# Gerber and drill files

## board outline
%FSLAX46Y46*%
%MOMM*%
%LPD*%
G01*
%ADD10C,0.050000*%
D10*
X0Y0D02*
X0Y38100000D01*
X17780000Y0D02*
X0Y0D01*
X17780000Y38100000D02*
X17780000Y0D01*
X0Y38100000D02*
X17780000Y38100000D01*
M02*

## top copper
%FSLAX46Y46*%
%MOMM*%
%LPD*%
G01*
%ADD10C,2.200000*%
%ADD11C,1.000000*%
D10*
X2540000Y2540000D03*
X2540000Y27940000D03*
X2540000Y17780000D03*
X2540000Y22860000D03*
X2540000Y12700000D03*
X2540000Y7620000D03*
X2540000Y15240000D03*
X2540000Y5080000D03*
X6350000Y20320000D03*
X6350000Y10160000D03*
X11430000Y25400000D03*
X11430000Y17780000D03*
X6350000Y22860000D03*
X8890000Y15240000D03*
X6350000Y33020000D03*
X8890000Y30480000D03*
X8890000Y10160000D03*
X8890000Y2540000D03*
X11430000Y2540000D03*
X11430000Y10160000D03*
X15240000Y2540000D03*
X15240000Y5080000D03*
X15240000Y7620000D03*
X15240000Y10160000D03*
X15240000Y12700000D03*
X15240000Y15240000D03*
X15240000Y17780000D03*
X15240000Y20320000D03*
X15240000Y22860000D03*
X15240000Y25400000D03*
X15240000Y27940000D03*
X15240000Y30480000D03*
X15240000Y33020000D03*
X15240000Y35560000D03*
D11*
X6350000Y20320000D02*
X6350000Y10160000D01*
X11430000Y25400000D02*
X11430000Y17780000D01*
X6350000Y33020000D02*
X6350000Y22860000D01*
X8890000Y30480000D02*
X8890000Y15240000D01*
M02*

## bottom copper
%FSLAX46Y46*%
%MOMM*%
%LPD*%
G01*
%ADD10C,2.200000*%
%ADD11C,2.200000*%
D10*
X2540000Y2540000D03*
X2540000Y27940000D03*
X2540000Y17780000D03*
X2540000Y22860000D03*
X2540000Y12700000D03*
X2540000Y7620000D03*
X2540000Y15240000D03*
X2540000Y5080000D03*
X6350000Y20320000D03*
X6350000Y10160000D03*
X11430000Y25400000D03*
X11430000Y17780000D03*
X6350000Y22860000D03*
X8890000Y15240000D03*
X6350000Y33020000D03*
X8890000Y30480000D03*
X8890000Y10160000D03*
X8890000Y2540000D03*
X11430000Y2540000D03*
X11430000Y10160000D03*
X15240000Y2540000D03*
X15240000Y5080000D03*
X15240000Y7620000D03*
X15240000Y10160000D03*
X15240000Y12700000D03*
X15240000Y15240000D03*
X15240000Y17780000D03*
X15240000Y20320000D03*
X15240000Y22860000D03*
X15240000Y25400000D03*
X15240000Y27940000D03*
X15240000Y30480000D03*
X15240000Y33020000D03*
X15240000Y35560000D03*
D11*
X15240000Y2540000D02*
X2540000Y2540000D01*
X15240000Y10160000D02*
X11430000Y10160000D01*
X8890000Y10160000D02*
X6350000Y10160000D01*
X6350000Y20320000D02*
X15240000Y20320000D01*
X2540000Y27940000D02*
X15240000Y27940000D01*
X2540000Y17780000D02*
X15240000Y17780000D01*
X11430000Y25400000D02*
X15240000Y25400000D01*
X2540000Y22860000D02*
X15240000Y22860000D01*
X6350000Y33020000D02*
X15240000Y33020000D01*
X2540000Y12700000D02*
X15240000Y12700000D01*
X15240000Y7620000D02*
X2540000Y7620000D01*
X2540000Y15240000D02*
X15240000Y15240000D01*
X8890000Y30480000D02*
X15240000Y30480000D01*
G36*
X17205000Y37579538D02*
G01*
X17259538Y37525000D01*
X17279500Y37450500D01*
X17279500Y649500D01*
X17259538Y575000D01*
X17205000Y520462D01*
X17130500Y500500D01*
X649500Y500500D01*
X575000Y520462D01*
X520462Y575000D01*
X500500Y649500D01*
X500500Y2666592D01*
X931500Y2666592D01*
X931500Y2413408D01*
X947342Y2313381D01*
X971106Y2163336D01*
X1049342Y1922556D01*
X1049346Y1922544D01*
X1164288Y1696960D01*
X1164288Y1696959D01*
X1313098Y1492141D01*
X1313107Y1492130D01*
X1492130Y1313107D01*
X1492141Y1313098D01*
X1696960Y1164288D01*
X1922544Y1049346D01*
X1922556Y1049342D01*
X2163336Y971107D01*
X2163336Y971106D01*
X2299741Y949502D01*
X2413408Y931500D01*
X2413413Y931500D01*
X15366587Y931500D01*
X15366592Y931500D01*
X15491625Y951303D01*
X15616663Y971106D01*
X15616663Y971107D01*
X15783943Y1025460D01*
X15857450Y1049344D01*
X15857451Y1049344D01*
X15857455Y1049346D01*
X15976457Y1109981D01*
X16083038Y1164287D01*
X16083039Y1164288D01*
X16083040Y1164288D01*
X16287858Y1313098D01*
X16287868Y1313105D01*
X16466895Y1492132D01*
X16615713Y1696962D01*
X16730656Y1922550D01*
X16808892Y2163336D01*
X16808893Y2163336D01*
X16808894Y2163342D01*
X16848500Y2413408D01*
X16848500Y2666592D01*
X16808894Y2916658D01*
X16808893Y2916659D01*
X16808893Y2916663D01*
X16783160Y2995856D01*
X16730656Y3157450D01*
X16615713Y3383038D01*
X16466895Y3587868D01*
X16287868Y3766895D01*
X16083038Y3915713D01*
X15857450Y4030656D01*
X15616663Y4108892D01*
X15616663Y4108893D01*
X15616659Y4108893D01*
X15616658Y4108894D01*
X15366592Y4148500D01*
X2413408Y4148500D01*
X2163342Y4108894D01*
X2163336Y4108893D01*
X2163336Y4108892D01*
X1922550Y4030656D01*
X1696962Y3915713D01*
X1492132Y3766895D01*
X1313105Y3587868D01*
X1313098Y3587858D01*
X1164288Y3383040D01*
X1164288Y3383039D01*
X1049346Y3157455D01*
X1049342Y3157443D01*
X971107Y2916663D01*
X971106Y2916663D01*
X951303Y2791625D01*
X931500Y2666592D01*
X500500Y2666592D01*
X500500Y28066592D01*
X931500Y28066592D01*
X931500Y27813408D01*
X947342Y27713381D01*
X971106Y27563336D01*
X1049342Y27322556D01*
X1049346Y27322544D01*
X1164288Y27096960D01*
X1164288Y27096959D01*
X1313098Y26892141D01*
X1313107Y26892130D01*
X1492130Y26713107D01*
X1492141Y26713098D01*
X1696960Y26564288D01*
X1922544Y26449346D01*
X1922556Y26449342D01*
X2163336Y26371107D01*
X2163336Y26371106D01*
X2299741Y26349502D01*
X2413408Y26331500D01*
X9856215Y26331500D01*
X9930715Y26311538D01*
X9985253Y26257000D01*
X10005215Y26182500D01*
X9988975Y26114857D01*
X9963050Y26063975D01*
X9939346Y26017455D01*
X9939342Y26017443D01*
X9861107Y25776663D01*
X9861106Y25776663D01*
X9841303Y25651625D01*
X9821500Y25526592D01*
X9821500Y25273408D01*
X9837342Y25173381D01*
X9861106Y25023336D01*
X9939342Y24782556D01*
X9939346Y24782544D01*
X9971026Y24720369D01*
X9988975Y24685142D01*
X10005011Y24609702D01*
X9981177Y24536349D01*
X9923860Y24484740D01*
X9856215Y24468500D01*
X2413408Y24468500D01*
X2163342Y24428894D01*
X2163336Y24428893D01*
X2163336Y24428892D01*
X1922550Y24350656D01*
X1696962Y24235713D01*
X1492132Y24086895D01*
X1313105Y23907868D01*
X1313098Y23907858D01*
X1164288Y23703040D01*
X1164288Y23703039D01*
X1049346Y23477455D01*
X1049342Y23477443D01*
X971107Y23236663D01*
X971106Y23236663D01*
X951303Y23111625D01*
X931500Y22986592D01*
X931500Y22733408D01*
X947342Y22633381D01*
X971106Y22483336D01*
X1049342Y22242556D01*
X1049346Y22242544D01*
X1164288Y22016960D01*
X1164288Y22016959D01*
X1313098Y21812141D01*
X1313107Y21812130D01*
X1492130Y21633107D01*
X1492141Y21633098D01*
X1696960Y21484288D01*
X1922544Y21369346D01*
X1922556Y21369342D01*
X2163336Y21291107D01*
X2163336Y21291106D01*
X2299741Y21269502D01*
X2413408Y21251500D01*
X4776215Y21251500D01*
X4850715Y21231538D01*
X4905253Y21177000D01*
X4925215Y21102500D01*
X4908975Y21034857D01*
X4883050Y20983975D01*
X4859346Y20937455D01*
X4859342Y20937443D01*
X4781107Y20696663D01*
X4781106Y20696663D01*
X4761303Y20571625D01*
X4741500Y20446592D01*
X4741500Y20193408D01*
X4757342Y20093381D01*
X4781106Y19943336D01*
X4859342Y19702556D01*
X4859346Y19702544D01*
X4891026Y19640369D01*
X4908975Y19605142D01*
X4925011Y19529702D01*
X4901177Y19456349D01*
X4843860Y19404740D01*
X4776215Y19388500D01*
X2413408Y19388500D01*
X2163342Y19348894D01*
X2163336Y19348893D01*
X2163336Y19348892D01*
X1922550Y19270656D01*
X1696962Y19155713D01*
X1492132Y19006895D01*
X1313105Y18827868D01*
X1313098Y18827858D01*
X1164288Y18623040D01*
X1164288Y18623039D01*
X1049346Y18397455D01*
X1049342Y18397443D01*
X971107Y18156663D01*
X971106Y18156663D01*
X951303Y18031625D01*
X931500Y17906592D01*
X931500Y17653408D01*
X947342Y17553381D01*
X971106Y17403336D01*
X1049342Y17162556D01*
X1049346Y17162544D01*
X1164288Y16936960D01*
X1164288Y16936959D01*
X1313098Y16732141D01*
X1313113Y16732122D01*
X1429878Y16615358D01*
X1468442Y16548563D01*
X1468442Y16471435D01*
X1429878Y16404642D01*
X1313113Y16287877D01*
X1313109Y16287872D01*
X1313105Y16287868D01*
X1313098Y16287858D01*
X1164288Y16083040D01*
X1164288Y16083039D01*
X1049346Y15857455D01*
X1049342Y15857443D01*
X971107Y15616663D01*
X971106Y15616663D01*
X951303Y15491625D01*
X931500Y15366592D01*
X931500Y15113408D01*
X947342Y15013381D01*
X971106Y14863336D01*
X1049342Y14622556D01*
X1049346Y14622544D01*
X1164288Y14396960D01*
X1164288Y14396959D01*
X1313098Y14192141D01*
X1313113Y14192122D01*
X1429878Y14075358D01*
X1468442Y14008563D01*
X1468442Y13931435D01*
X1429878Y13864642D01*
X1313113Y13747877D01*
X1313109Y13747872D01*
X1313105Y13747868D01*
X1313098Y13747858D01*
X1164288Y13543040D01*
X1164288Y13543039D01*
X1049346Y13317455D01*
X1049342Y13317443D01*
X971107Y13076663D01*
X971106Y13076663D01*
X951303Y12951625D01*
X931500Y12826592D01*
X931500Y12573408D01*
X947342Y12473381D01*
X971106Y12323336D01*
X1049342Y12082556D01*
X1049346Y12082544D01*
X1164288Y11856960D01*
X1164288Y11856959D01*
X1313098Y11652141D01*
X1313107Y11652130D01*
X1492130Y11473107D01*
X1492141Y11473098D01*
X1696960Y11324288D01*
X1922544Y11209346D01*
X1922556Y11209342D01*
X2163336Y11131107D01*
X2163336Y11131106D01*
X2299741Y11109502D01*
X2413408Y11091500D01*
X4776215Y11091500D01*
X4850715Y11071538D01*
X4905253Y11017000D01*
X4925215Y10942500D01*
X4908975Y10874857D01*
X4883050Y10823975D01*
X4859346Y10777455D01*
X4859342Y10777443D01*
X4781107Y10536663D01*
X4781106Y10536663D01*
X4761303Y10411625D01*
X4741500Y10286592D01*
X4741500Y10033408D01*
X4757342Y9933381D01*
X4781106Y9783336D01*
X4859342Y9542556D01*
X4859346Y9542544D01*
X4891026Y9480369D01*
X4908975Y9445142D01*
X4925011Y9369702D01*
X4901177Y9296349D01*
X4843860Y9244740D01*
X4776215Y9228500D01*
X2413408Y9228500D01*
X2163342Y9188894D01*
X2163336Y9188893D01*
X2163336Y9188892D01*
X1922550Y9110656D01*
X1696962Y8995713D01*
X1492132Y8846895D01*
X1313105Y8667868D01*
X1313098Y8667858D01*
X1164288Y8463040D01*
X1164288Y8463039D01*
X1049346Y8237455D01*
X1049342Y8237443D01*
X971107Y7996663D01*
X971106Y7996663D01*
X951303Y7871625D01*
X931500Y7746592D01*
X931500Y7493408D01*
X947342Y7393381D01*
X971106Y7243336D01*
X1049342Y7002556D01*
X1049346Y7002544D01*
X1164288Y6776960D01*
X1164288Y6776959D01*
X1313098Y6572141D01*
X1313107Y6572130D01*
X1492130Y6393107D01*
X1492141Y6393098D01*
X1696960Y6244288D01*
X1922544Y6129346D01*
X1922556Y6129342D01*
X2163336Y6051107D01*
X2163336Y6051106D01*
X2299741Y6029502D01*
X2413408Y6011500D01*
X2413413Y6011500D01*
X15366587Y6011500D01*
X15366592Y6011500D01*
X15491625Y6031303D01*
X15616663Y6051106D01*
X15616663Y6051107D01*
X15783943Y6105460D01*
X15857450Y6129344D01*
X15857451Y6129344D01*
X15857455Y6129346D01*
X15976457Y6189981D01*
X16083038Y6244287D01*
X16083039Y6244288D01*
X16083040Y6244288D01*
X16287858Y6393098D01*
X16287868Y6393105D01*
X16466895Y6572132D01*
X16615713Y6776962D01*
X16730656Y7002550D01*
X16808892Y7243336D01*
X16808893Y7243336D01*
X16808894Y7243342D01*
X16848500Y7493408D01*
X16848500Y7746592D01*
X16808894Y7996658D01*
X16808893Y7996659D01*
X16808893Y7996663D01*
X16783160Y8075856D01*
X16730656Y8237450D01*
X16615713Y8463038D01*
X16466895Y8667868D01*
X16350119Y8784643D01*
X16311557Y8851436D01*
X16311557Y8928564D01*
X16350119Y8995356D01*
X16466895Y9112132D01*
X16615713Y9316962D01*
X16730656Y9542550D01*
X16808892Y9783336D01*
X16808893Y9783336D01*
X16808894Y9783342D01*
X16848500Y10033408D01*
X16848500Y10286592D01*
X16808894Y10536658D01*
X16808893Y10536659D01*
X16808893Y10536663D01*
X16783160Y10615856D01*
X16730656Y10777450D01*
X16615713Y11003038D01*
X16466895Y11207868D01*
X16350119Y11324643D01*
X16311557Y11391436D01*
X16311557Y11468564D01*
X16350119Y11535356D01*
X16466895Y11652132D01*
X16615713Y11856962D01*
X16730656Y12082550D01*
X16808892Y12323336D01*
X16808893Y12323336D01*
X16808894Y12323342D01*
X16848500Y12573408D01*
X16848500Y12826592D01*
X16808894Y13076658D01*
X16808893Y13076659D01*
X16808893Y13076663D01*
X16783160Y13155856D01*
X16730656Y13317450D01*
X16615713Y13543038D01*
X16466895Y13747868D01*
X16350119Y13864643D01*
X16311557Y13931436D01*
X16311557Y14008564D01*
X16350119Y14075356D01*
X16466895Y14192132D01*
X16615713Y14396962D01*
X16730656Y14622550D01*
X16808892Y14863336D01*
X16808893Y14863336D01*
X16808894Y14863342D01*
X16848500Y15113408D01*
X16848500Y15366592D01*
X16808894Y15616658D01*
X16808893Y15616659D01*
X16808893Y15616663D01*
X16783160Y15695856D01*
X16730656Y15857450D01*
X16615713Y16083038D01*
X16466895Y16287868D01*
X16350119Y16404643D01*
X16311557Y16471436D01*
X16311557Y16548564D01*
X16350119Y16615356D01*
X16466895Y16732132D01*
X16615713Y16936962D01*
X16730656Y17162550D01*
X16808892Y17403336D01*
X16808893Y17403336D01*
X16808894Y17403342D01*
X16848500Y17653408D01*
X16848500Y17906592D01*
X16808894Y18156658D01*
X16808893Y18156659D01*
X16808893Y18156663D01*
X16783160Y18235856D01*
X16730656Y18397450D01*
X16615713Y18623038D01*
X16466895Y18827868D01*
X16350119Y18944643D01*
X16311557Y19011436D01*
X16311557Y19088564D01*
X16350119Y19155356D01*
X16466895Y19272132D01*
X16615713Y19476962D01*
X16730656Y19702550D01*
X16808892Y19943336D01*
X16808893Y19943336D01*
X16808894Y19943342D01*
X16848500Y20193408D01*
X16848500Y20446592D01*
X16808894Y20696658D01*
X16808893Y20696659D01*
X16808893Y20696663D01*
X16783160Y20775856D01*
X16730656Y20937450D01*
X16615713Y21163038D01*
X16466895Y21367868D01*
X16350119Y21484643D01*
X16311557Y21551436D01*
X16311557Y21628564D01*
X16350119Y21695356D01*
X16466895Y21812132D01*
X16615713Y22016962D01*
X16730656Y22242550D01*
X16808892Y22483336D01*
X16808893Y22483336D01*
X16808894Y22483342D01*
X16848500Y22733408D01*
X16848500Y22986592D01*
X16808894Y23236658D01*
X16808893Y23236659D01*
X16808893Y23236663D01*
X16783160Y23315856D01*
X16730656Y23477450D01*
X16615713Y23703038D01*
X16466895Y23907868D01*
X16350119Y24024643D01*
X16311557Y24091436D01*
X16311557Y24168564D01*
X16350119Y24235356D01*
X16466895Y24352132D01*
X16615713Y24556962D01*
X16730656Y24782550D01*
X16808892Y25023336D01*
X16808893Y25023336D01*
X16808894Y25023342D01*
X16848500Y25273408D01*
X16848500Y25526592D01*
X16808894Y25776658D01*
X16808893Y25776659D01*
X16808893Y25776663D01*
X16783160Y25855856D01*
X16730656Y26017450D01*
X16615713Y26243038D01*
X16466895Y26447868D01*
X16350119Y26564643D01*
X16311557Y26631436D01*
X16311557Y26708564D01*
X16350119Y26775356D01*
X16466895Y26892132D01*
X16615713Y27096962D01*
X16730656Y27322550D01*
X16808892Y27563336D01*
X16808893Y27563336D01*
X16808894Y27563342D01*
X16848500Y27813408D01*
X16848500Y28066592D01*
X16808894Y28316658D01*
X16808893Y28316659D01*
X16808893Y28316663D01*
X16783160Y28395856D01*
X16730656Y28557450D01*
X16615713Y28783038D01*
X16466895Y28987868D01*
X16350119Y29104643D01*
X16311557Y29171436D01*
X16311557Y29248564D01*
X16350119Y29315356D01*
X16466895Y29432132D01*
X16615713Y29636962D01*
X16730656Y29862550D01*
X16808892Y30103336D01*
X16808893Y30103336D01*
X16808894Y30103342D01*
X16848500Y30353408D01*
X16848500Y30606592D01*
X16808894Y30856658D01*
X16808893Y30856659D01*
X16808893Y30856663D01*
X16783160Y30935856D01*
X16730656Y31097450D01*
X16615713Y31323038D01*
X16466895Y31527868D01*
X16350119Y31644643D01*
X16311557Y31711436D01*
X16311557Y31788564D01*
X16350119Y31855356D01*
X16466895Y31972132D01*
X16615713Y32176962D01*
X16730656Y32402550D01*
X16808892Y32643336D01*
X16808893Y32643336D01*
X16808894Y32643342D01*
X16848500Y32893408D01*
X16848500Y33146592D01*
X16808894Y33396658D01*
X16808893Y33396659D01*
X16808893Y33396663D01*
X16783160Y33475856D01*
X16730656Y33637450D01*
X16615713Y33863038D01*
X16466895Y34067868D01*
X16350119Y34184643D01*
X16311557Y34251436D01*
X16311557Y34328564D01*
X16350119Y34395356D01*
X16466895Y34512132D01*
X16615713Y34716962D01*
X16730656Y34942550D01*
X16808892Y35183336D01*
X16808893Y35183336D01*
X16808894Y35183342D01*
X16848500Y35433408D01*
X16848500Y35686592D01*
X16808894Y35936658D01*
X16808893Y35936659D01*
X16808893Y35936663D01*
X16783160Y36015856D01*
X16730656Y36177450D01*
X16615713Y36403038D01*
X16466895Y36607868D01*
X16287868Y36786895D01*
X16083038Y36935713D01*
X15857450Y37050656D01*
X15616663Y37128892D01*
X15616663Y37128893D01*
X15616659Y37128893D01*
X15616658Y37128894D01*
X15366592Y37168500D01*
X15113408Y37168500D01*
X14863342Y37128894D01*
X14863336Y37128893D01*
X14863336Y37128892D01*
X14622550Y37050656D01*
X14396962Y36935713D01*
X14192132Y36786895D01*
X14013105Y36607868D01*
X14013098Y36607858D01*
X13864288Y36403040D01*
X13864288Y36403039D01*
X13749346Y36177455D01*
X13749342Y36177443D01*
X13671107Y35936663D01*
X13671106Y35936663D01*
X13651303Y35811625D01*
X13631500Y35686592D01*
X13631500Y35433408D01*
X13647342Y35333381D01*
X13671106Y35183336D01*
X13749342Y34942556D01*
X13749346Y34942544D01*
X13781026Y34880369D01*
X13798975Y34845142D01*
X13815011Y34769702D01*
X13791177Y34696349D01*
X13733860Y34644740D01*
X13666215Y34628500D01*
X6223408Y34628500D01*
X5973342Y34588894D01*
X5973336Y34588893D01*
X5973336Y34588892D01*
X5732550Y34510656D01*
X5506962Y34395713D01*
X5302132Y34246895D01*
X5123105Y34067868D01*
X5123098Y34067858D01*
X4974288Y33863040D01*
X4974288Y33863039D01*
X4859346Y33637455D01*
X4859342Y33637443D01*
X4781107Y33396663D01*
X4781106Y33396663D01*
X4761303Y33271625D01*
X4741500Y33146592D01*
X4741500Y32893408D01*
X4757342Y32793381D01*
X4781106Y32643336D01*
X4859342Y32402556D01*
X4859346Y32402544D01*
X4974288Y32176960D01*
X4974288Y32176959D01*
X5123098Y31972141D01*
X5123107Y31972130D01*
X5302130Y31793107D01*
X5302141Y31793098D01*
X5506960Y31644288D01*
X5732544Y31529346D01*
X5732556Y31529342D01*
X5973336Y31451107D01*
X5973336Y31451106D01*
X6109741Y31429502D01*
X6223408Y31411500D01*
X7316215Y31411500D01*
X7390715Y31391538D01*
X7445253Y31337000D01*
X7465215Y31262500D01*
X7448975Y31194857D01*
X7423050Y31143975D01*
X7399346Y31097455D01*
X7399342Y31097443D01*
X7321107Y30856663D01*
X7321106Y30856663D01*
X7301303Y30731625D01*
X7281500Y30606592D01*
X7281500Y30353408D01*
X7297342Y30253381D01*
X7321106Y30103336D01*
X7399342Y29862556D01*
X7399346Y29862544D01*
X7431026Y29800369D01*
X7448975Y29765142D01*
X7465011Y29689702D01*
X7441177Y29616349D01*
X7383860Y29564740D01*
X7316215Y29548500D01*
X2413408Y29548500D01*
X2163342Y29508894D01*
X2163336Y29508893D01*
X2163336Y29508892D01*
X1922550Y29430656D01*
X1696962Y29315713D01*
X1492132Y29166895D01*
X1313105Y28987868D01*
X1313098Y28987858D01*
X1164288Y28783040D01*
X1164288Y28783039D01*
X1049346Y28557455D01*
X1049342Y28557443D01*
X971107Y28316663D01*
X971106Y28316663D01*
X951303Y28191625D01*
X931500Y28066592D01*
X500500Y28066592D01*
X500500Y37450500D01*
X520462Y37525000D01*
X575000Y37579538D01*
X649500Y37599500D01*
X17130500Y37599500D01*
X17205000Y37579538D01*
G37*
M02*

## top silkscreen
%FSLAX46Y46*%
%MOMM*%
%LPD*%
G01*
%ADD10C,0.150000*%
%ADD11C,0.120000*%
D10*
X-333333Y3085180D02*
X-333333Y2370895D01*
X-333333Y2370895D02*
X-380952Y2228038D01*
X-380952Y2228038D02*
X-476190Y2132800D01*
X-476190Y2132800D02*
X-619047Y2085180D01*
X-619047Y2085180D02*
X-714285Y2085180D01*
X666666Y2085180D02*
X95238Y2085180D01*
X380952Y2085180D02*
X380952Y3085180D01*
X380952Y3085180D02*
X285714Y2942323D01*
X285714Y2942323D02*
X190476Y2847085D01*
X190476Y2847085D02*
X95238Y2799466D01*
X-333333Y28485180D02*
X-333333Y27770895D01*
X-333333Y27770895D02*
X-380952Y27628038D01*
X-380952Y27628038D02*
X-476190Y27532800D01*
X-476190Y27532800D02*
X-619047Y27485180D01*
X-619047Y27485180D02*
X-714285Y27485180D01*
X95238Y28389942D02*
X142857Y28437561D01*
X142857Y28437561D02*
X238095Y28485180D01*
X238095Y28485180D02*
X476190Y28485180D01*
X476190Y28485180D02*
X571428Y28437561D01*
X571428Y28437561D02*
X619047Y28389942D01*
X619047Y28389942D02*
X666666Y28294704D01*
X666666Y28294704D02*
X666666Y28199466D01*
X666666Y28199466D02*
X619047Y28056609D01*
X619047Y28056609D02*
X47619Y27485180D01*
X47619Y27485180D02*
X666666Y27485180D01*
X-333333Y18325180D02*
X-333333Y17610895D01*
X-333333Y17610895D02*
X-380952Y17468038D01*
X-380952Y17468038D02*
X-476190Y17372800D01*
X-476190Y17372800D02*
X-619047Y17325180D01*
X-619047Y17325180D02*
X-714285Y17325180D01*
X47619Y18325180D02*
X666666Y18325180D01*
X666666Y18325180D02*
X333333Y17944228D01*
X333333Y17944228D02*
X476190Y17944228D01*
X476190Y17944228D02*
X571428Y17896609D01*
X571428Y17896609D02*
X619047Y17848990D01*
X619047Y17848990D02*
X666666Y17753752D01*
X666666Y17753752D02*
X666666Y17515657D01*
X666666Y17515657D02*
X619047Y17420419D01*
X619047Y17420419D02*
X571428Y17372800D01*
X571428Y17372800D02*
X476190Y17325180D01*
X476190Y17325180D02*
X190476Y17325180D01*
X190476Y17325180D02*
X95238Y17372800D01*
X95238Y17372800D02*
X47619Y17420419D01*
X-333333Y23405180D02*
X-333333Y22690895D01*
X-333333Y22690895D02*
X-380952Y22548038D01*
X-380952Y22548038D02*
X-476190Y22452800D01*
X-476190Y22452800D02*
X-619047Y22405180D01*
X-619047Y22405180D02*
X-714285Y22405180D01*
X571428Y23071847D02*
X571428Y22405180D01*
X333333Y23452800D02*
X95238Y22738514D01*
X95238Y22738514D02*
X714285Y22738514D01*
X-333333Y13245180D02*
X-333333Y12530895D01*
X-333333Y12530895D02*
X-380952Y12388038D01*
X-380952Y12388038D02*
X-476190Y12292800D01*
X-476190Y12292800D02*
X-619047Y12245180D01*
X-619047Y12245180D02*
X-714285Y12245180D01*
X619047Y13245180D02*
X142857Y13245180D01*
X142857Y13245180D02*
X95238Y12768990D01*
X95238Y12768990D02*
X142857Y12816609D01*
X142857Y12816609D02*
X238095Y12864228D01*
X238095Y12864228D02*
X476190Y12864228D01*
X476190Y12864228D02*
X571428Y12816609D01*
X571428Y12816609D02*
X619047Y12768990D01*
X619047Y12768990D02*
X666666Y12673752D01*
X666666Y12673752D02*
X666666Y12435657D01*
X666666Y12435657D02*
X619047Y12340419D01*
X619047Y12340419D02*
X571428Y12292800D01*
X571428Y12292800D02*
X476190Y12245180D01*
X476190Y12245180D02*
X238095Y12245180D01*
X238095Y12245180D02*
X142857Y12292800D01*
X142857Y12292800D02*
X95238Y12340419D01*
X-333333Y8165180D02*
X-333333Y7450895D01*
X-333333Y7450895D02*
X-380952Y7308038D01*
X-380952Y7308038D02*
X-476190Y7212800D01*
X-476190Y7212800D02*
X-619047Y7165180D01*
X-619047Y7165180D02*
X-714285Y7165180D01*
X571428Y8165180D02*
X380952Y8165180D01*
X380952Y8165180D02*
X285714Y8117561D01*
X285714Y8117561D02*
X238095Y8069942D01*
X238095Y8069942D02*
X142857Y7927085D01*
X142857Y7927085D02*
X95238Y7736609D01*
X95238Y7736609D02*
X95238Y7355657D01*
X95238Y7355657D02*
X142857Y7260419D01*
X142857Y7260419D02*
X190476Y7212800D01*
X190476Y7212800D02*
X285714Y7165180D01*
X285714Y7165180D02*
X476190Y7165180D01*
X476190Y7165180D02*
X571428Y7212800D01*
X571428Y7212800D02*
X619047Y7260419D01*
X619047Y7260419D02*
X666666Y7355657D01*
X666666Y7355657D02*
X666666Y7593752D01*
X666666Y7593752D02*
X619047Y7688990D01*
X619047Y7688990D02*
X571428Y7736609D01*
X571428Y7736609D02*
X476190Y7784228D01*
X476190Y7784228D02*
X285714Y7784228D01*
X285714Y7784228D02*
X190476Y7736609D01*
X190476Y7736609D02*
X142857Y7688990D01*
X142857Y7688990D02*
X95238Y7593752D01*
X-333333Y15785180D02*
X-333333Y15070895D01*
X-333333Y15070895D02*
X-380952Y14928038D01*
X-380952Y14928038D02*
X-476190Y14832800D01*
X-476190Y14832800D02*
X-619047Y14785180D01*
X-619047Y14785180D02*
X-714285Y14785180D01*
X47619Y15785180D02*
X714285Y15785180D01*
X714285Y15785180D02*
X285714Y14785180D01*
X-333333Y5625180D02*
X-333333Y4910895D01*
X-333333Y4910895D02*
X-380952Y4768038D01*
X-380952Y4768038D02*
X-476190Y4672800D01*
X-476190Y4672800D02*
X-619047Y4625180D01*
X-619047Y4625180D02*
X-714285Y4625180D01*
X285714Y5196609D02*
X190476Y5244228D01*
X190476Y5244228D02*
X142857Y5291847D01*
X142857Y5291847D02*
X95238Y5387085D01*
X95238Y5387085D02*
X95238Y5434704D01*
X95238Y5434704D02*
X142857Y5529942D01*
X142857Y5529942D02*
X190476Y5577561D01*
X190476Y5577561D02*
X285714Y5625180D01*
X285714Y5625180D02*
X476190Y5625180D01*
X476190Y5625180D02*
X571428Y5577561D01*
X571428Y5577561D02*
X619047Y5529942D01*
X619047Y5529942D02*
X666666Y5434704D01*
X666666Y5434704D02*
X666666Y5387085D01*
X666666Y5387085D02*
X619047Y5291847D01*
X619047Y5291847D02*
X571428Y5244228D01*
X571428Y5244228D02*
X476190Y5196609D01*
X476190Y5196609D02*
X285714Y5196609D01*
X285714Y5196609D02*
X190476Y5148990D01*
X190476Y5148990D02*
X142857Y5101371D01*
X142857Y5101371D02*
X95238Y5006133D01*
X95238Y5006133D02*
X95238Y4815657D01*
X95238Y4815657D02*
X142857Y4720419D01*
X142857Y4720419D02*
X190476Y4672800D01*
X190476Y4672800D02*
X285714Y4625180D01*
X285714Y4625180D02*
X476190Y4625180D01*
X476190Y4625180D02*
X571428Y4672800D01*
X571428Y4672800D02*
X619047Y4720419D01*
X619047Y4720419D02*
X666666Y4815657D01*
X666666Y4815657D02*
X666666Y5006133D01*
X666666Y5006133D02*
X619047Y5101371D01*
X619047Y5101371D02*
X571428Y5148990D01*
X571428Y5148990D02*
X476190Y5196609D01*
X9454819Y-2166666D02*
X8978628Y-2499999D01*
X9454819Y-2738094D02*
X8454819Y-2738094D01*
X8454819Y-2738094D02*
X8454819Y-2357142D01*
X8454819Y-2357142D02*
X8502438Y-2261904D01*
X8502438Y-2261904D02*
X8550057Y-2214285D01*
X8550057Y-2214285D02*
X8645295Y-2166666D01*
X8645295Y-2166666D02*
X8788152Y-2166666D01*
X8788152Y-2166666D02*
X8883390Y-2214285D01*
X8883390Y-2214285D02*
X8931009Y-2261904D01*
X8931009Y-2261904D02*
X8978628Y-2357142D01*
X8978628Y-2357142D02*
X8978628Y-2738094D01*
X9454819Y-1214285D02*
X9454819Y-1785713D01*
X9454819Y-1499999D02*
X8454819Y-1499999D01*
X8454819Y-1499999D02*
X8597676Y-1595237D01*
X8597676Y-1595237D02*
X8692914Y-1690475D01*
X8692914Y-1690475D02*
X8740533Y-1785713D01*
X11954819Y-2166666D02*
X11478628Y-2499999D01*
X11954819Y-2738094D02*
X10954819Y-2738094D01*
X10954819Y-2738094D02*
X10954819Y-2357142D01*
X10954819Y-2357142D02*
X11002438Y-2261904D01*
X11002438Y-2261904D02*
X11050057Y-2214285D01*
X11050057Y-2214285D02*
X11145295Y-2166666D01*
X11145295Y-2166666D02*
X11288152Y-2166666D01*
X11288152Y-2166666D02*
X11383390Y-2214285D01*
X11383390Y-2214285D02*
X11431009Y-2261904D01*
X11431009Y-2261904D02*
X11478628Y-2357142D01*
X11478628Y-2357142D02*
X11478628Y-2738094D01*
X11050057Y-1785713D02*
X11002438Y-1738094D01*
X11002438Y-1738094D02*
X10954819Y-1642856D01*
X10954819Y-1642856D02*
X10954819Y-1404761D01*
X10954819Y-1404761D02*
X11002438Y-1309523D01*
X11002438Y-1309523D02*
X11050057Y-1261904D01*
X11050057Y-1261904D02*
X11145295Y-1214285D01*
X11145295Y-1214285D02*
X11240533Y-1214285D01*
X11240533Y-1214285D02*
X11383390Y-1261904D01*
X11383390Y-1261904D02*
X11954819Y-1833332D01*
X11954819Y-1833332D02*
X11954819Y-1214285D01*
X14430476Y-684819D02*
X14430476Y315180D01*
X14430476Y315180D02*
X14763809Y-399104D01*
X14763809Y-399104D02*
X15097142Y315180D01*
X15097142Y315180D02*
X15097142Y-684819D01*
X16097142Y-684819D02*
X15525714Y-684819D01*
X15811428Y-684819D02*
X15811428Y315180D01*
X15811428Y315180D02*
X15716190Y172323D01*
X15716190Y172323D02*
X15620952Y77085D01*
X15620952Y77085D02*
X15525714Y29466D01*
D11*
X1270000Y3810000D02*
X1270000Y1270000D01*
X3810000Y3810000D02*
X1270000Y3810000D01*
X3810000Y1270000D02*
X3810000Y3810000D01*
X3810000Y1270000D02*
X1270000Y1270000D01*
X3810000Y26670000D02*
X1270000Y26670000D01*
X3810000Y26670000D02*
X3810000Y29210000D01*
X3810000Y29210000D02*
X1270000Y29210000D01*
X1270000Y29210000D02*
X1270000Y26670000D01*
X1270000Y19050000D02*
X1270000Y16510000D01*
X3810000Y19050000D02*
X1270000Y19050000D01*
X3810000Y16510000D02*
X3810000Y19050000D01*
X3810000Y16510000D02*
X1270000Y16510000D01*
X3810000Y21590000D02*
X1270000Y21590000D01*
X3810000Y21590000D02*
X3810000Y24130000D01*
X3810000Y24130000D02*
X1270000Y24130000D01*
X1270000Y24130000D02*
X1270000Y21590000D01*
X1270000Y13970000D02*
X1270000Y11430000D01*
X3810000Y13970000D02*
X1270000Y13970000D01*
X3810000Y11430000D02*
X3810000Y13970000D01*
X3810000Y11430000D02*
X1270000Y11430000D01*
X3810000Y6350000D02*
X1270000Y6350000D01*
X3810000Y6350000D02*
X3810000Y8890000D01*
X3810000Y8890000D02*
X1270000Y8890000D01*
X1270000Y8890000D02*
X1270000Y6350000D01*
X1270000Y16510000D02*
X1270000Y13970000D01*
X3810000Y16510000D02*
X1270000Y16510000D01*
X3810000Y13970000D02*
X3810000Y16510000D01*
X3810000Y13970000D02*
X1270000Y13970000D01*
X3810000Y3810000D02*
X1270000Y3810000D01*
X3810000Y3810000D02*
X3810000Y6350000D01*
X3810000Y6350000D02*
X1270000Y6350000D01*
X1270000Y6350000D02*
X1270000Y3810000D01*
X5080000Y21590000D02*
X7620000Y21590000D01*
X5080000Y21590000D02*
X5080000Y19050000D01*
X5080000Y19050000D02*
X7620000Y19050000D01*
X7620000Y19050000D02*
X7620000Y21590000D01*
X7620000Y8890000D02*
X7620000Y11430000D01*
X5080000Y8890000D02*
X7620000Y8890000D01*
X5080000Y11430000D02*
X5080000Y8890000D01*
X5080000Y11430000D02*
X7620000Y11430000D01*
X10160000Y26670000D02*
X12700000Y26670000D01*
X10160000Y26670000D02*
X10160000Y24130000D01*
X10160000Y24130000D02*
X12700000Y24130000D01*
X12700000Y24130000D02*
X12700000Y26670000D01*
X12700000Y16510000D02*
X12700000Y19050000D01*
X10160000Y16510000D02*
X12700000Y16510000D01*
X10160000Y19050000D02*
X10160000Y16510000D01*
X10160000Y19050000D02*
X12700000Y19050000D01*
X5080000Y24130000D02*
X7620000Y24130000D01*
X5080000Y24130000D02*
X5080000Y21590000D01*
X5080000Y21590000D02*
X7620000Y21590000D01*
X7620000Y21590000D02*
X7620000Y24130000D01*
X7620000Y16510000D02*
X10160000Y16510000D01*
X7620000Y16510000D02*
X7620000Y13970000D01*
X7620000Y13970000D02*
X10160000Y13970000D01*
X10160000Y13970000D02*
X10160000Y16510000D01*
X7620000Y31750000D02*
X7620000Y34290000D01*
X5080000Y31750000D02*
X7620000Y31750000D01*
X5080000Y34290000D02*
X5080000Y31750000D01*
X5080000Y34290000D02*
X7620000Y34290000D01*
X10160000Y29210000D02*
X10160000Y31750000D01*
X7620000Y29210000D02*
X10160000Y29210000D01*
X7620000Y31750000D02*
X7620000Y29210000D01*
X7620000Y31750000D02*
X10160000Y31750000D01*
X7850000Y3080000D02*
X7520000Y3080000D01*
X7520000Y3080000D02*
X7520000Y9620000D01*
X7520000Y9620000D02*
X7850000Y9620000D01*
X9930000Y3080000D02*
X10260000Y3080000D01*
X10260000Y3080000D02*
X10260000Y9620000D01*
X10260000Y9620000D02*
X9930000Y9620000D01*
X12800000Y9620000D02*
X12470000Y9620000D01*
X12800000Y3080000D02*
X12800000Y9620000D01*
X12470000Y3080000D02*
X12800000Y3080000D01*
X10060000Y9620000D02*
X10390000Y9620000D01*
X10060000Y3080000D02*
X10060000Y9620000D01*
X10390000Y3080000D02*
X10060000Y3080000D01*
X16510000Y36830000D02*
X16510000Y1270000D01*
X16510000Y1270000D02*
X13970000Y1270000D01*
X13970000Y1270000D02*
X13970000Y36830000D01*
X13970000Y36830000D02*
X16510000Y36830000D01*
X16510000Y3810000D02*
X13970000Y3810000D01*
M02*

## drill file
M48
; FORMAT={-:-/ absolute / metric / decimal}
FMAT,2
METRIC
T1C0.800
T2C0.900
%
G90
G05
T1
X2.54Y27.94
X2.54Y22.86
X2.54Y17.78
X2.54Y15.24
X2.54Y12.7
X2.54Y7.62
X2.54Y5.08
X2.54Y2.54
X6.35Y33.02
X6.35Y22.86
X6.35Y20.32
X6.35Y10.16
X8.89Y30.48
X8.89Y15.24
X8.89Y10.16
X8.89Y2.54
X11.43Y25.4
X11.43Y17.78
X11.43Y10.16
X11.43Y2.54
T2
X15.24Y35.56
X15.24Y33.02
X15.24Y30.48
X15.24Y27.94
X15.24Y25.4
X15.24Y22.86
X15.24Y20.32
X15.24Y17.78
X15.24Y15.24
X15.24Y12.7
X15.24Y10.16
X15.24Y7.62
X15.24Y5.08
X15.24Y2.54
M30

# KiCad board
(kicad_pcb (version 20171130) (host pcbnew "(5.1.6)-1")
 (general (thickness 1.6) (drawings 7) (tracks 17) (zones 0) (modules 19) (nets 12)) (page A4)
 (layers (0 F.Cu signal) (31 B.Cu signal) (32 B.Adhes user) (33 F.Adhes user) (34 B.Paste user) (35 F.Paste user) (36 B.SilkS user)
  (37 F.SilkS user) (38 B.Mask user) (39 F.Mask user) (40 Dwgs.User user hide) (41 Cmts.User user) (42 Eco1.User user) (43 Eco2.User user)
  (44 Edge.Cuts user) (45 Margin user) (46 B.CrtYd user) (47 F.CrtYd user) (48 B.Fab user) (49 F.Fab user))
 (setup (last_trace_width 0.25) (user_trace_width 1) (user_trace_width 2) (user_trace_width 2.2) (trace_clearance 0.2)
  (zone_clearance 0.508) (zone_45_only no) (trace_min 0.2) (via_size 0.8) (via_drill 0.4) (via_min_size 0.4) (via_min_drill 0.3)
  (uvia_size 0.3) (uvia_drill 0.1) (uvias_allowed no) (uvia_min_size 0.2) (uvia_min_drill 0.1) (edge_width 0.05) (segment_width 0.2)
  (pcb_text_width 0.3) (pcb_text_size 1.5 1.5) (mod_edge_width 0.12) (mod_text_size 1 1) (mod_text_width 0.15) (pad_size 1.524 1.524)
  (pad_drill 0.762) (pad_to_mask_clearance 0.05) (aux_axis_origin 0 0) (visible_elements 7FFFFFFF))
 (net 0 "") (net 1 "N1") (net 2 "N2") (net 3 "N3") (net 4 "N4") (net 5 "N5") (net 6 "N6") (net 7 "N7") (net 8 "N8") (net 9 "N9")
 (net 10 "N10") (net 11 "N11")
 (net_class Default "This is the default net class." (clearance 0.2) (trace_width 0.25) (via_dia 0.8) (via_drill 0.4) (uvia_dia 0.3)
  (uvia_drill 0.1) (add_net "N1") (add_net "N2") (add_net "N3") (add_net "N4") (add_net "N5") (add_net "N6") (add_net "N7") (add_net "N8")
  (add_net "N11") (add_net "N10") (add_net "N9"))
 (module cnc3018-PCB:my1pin (layer F.Cu) (at 2.54 -2.54 180)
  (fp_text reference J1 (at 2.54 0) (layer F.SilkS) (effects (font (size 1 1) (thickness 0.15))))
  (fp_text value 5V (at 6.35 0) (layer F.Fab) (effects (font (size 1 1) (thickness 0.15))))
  (fp_line (start 1.27 1.27) (end 1.27 -1.27) (layer F.SilkS) (width 0.12))
  (fp_line (start -1.27 1.27) (end 1.27 1.27) (layer F.SilkS) (width 0.12))
  (fp_line (start -1.27 -1.27) (end -1.27 1.27) (layer F.SilkS) (width 0.12))
  (fp_line (start -1.27 -1.27) (end 1.27 -1.27) (layer F.SilkS) (width 0.12))
  (pad 1 thru_hole circle (at 0 0 180) (size 2.2 2.2) (drill 0.8) (layers *.Cu *.Mask) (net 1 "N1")))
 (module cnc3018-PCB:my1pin (layer F.Cu) (at 2.54 -27.94 180)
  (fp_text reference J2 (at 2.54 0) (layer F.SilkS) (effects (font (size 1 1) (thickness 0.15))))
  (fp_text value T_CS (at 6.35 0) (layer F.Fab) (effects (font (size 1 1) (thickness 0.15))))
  (fp_line (start -1.27 -1.27) (end 1.27 -1.27) (layer F.SilkS) (width 0.12))
  (fp_line (start -1.27 -1.27) (end -1.27 1.27) (layer F.SilkS) (width 0.12))
  (fp_line (start -1.27 1.27) (end 1.27 1.27) (layer F.SilkS) (width 0.12))
  (fp_line (start 1.27 1.27) (end 1.27 -1.27) (layer F.SilkS) (width 0.12))
  (pad 1 thru_hole circle (at 0 0 180) (size 2.2 2.2) (drill 0.8) (layers *.Cu *.Mask) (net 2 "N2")))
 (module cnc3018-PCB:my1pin (layer F.Cu) (at 2.54 -17.78 180)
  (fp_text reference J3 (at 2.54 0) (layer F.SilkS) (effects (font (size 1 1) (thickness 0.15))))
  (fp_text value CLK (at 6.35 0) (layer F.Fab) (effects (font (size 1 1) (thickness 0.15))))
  (fp_line (start 1.27 1.27) (end 1.27 -1.27) (layer F.SilkS) (width 0.12))
  (fp_line (start -1.27 1.27) (end 1.27 1.27) (layer F.SilkS) (width 0.12))
  (fp_line (start -1.27 -1.27) (end -1.27 1.27) (layer F.SilkS) (width 0.12))
  (fp_line (start -1.27 -1.27) (end 1.27 -1.27) (layer F.SilkS) (width 0.12))
  (pad 1 thru_hole circle (at 0 0 180) (size 2.2 2.2) (drill 0.8) (layers *.Cu *.Mask) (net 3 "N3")))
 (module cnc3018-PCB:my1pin (layer F.Cu) (at 2.54 -22.86 180)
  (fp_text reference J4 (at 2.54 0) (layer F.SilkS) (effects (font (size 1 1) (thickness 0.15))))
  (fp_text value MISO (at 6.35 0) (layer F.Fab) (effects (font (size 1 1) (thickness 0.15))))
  (fp_line (start -1.27 -1.27) (end 1.27 -1.27) (layer F.SilkS) (width 0.12))
  (fp_line (start -1.27 -1.27) (end -1.27 1.27) (layer F.SilkS) (width 0.12))
  (fp_line (start -1.27 1.27) (end 1.27 1.27) (layer F.SilkS) (width 0.12))
  (fp_line (start 1.27 1.27) (end 1.27 -1.27) (layer F.SilkS) (width 0.12))
  (pad 1 thru_hole circle (at 0 0 180) (size 2.2 2.2) (drill 0.8) (layers *.Cu *.Mask) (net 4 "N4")))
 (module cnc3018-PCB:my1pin (layer F.Cu) (at 2.54 -12.7 180)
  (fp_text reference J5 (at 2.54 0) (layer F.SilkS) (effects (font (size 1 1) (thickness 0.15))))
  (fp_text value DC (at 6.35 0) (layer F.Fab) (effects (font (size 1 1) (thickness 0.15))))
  (fp_line (start 1.27 1.27) (end 1.27 -1.27) (layer F.SilkS) (width 0.12))
  (fp_line (start -1.27 1.27) (end 1.27 1.27) (layer F.SilkS) (width 0.12))
  (fp_line (start -1.27 -1.27) (end -1.27 1.27) (layer F.SilkS) (width 0.12))
  (fp_line (start -1.27 -1.27) (end 1.27 -1.27) (layer F.SilkS) (width 0.12))
  (pad 1 thru_hole circle (at 0 0 180) (size 2.2 2.2) (drill 0.8) (layers *.Cu *.Mask) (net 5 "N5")))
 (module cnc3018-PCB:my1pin (layer F.Cu) (at 2.54 -7.62 180)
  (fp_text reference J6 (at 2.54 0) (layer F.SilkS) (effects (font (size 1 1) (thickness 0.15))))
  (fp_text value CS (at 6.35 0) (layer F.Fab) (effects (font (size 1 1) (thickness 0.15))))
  (fp_line (start -1.27 -1.27) (end 1.27 -1.27) (layer F.SilkS) (width 0.12))
  (fp_line (start -1.27 -1.27) (end -1.27 1.27) (layer F.SilkS) (width 0.12))
  (fp_line (start -1.27 1.27) (end 1.27 1.27) (layer F.SilkS) (width 0.12))
  (fp_line (start 1.27 1.27) (end 1.27 -1.27) (layer F.SilkS) (width 0.12))
  (pad 1 thru_hole circle (at 0 0 180) (size 2.2 2.2) (drill 0.8) (layers *.Cu *.Mask) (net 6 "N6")))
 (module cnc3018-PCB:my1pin (layer F.Cu) (at 2.54 -15.24 180)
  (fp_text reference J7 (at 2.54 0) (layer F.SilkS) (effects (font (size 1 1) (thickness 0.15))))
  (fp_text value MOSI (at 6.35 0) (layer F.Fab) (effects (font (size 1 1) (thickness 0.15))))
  (fp_line (start 1.27 1.27) (end 1.27 -1.27) (layer F.SilkS) (width 0.12))
  (fp_line (start -1.27 1.27) (end 1.27 1.27) (layer F.SilkS) (width 0.12))
  (fp_line (start -1.27 -1.27) (end -1.27 1.27) (layer F.SilkS) (width 0.12))
  (fp_line (start -1.27 -1.27) (end 1.27 -1.27) (layer F.SilkS) (width 0.12))
  (pad 1 thru_hole circle (at 0 0 180) (size 2.2 2.2) (drill 0.8) (layers *.Cu *.Mask) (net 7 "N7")))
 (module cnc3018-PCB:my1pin (layer F.Cu) (at 2.54 -5.08 180)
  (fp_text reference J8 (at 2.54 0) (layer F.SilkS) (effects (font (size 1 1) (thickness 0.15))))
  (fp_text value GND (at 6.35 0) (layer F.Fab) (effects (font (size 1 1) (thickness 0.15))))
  (fp_line (start -1.27 -1.27) (end 1.27 -1.27) (layer F.SilkS) (width 0.12))
  (fp_line (start -1.27 -1.27) (end -1.27 1.27) (layer F.SilkS) (width 0.12))
  (fp_line (start -1.27 1.27) (end 1.27 1.27) (layer F.SilkS) (width 0.12))
  (fp_line (start 1.27 1.27) (end 1.27 -1.27) (layer F.SilkS) (width 0.12))
  (pad 1 thru_hole circle (at 0 0 180) (size 2.2 2.2) (drill 0.8) (layers *.Cu *.Mask) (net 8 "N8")))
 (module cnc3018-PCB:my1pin (layer F.Cu) (at 6.35 -20.32)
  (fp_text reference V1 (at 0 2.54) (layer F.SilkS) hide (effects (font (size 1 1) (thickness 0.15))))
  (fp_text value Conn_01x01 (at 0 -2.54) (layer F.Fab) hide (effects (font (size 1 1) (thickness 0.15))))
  (fp_line (start -1.27 -1.27) (end 1.27 -1.27) (layer F.SilkS) (width 0.12))
  (fp_line (start -1.27 -1.27) (end -1.27 1.27) (layer F.SilkS) (width 0.12))
  (fp_line (start -1.27 1.27) (end 1.27 1.27) (layer F.SilkS) (width 0.12))
  (fp_line (start 1.27 1.27) (end 1.27 -1.27) (layer F.SilkS) (width 0.12))
  (pad 1 thru_hole circle (at 0 0) (size 2.2 2.2) (drill 0.8) (layers *.Cu *.Mask) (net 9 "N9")))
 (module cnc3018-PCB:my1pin (layer F.Cu) (at 6.35 -10.16)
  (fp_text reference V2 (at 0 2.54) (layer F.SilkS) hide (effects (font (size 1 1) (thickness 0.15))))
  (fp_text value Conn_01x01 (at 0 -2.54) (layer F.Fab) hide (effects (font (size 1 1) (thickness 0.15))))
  (fp_line (start 1.27 1.27) (end 1.27 -1.27) (layer F.SilkS) (width 0.12))
  (fp_line (start -1.27 1.27) (end 1.27 1.27) (layer F.SilkS) (width 0.12))
  (fp_line (start -1.27 -1.27) (end -1.27 1.27) (layer F.SilkS) (width 0.12))
  (fp_line (start -1.27 -1.27) (end 1.27 -1.27) (layer F.SilkS) (width 0.12))
  (pad 1 thru_hole circle (at 0 0) (size 2.2 2.2) (drill 0.8) (layers *.Cu *.Mask) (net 9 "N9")))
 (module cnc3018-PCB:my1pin (layer F.Cu) (at 11.43 -25.4)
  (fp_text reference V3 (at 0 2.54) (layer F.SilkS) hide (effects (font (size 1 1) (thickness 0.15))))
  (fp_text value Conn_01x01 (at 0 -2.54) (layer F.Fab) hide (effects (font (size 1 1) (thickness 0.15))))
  (fp_line (start -1.27 -1.27) (end 1.27 -1.27) (layer F.SilkS) (width 0.12))
  (fp_line (start -1.27 -1.27) (end -1.27 1.27) (layer F.SilkS) (width 0.12))
  (fp_line (start -1.27 1.27) (end 1.27 1.27) (layer F.SilkS) (width 0.12))
  (fp_line (start 1.27 1.27) (end 1.27 -1.27) (layer F.SilkS) (width 0.12))
  (pad 1 thru_hole circle (at 0 0) (size 2.2 2.2) (drill 0.8) (layers *.Cu *.Mask) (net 3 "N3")))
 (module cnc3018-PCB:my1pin (layer F.Cu) (at 11.43 -17.78)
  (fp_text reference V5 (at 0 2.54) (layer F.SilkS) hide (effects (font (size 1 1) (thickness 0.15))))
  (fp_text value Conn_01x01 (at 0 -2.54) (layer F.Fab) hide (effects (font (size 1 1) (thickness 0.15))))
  (fp_line (start 1.27 1.27) (end 1.27 -1.27) (layer F.SilkS) (width 0.12))
  (fp_line (start -1.27 1.27) (end 1.27 1.27) (layer F.SilkS) (width 0.12))
  (fp_line (start -1.27 -1.27) (end -1.27 1.27) (layer F.SilkS) (width 0.12))
  (fp_line (start -1.27 -1.27) (end 1.27 -1.27) (layer F.SilkS) (width 0.12))
  (pad 1 thru_hole circle (at 0 0) (size 2.2 2.2) (drill 0.8) (layers *.Cu *.Mask) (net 3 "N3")))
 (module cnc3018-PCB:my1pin (layer F.Cu) (at 6.35 -22.86)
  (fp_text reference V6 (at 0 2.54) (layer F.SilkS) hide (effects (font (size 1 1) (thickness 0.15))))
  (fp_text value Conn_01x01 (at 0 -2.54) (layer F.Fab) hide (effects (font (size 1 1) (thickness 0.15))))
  (fp_line (start -1.27 -1.27) (end 1.27 -1.27) (layer F.SilkS) (width 0.12))
  (fp_line (start -1.27 -1.27) (end -1.27 1.27) (layer F.SilkS) (width 0.12))
  (fp_line (start -1.27 1.27) (end 1.27 1.27) (layer F.SilkS) (width 0.12))
  (fp_line (start 1.27 1.27) (end 1.27 -1.27) (layer F.SilkS) (width 0.12))
  (pad 1 thru_hole circle (at 0 0) (size 2.2 2.2) (drill 0.8) (layers *.Cu *.Mask) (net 4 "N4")))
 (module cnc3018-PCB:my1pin (layer F.Cu) (at 8.89 -15.24)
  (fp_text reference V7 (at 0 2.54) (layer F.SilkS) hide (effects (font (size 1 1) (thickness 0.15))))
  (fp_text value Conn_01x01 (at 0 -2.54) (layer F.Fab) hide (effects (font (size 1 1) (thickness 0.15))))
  (fp_line (start -1.27 -1.27) (end 1.27 -1.27) (layer F.SilkS) (width 0.12))
  (fp_line (start -1.27 -1.27) (end -1.27 1.27) (layer F.SilkS) (width 0.12))
  (fp_line (start -1.27 1.27) (end 1.27 1.27) (layer F.SilkS) (width 0.12))
  (fp_line (start 1.27 1.27) (end 1.27 -1.27) (layer F.SilkS) (width 0.12))
  (pad 1 thru_hole circle (at 0 0) (size 2.2 2.2) (drill 0.8) (layers *.Cu *.Mask) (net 7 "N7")))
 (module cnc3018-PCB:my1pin (layer F.Cu) (at 6.35 -33.02)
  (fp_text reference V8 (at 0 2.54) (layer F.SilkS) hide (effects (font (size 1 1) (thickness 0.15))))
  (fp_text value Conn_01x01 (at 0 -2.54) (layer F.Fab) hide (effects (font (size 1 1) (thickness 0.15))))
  (fp_line (start 1.27 1.27) (end 1.27 -1.27) (layer F.SilkS) (width 0.12))
  (fp_line (start -1.27 1.27) (end 1.27 1.27) (layer F.SilkS) (width 0.12))
  (fp_line (start -1.27 -1.27) (end -1.27 1.27) (layer F.SilkS) (width 0.12))
  (fp_line (start -1.27 -1.27) (end 1.27 -1.27) (layer F.SilkS) (width 0.12))
  (pad 1 thru_hole circle (at 0 0) (size 2.2 2.2) (drill 0.8) (layers *.Cu *.Mask) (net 4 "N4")))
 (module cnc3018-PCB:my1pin (layer F.Cu) (at 8.89 -30.48)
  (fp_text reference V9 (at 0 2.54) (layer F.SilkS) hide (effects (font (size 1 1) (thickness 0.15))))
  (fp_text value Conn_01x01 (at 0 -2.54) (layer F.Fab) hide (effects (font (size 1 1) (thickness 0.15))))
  (fp_line (start 1.27 1.27) (end 1.27 -1.27) (layer F.SilkS) (width 0.12))
  (fp_line (start -1.27 1.27) (end 1.27 1.27) (layer F.SilkS) (width 0.12))
  (fp_line (start -1.27 -1.27) (end -1.27 1.27) (layer F.SilkS) (width 0.12))
  (fp_line (start -1.27 -1.27) (end 1.27 -1.27) (layer F.SilkS) (width 0.12))
  (pad 1 thru_hole circle (at 0 0) (size 2.2 2.2) (drill 0.8) (layers *.Cu *.Mask) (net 7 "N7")))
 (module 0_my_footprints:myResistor (layer F.Cu) (at 8.89 -2.54 90)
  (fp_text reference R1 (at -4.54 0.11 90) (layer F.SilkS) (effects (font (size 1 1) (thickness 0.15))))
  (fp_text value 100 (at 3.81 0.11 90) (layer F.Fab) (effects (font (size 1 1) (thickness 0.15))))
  (fp_line (start 0.54 -1.04) (end 0.54 -1.37) (layer F.SilkS) (width 0.12))
  (fp_line (start 0.54 -1.37) (end 7.08 -1.37) (layer F.SilkS) (width 0.12))
  (fp_line (start 7.08 -1.37) (end 7.08 -1.04) (layer F.SilkS) (width 0.12))
  (fp_line (start 0.54 1.04) (end 0.54 1.37) (layer F.SilkS) (width 0.12))
  (fp_line (start 0.54 1.37) (end 7.08 1.37) (layer F.SilkS) (width 0.12))
  (fp_line (start 7.08 1.37) (end 7.08 1.04) (layer F.SilkS) (width 0.12))
  (pad 2 thru_hole circle (at 7.62 0 90) (size 2.2 2.2) (drill 0.8) (layers *.Cu *.Mask) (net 9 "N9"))
  (pad 1 thru_hole circle (at 0 0 90) (size 2.2 2.2) (drill 0.8) (layers *.Cu *.Mask) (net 1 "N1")))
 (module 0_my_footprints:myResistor (layer F.Cu) (at 11.43 -2.54 90)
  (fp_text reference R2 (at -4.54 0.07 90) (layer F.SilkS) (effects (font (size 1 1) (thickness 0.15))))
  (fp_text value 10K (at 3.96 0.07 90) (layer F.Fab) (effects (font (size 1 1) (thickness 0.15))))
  (fp_line (start 7.08 1.37) (end 7.08 1.04) (layer F.SilkS) (width 0.12))
  (fp_line (start 0.54 1.37) (end 7.08 1.37) (layer F.SilkS) (width 0.12))
  (fp_line (start 0.54 1.04) (end 0.54 1.37) (layer F.SilkS) (width 0.12))
  (fp_line (start 7.08 -1.37) (end 7.08 -1.04) (layer F.SilkS) (width 0.12))
  (fp_line (start 0.54 -1.37) (end 7.08 -1.37) (layer F.SilkS) (width 0.12))
  (fp_line (start 0.54 -1.04) (end 0.54 -1.37) (layer F.SilkS) (width 0.12))
  (pad 1 thru_hole circle (at 0 0 90) (size 2.2 2.2) (drill 0.8) (layers *.Cu *.Mask) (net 1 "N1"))
  (pad 2 thru_hole circle (at 7.62 0 90) (size 2.2 2.2) (drill 0.8) (layers *.Cu *.Mask) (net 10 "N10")))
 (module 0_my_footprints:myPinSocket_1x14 (layer F.Cu) (at 15.24 -2.54 180)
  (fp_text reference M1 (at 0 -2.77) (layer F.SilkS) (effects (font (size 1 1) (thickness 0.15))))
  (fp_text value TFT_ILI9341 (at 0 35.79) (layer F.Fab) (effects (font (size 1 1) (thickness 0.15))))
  (fp_line (start -1.27 34.29) (end -1.27 -1.27) (layer F.SilkS) (width 0.12))
  (fp_line (start -1.27 -1.27) (end 1.27 -1.27) (layer F.SilkS) (width 0.12))
  (fp_line (start 1.27 -1.27) (end 1.27 34.29) (layer F.SilkS) (width 0.12))
  (fp_line (start 1.27 34.29) (end -1.27 34.29) (layer F.SilkS) (width 0.12))
  (fp_line (start -1.27 1.27) (end 1.27 1.27) (layer F.SilkS) (width 0.12))
  (pad 1 thru_hole circle (at 0 0 180) (size 2.2 2.2) (drill 0.9) (layers *.Cu *.Mask) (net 1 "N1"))
  (pad 2 thru_hole circle (at 0 2.54 180) (size 2.2 2.2) (drill 0.9) (layers *.Cu *.Mask) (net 8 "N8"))
  (pad 3 thru_hole circle (at 0 5.08 180) (size 2.2 2.2) (drill 0.9) (layers *.Cu *.Mask) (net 6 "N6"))
  (pad 4 thru_hole circle (at 0 7.62 180) (size 2.2 2.2) (drill 0.9) (layers *.Cu *.Mask) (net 10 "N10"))
  (pad 5 thru_hole circle (at 0 10.16 180) (size 2.2 2.2) (drill 0.9) (layers *.Cu *.Mask) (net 5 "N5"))
  (pad 6 thru_hole circle (at 0 12.7 180) (size 2.2 2.2) (drill 0.9) (layers *.Cu *.Mask) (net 7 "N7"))
  (pad 7 thru_hole circle (at 0 15.24 180) (size 2.2 2.2) (drill 0.9) (layers *.Cu *.Mask) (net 3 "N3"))
  (pad 8 thru_hole circle (at 0 17.78 180) (size 2.2 2.2) (drill 0.9) (layers *.Cu *.Mask) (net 9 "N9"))
  (pad 9 thru_hole circle (at 0 20.32 180) (size 2.2 2.2) (drill 0.9) (layers *.Cu *.Mask) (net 4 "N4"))
  (pad 10 thru_hole circle (at 0 22.86 180) (size 2.2 2.2) (drill 0.9) (layers *.Cu *.Mask) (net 3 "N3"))
  (pad 11 thru_hole circle (at 0 25.4 180) (size 2.2 2.2) (drill 0.9) (layers *.Cu *.Mask) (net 2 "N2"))
  (pad 12 thru_hole circle (at 0 27.94 180) (size 2.2 2.2) (drill 0.9) (layers *.Cu *.Mask) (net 7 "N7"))
  (pad 13 thru_hole circle (at 0 30.48 180) (size 2.2 2.2) (drill 0.9) (layers *.Cu *.Mask) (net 4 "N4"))
  (pad 14 thru_hole circle (at 0 33.02 180) (size 2.2 2.2) (drill 0.9) (layers *.Cu *.Mask) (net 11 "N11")))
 (gr_line (start 0 0) (end 0 -38.1) (layer Edge.Cuts) (width 0.05))
 (gr_line (start 17.78 0) (end 0 0) (layer Edge.Cuts) (width 0.05))
 (gr_line (start 17.78 -38.1) (end 17.78 0) (layer Edge.Cuts) (width 0.05))
 (gr_line (start 0 -38.1) (end 17.78 -38.1) (layer Edge.Cuts) (width 0.05))
 (segment (start 15.24 -2.54) (end 2.54 -2.54) (width 2.2) (layer B.Cu) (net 1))
 (segment (start 15.24 -10.16) (end 11.43 -10.16) (width 2.2) (layer B.Cu) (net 10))
 (segment (start 6.35 -20.32) (end 6.35 -10.16) (width 1) (layer F.Cu) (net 9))
 (segment (start 8.89 -10.16) (end 6.35 -10.16) (width 2.2) (layer B.Cu) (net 9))
 (segment (start 6.35 -20.32) (end 15.24 -20.32) (width 2.2) (layer B.Cu) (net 9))
 (segment (start 2.54 -27.94) (end 15.24 -27.94) (width 2.2) (layer B.Cu) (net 2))
 (segment (start 11.43 -25.4) (end 11.43 -17.78) (width 1) (layer F.Cu) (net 3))
 (segment (start 2.54 -17.78) (end 15.24 -17.78) (width 2.2) (layer B.Cu) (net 3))
 (segment (start 11.43 -25.4) (end 15.24 -25.4) (width 2.2) (layer B.Cu) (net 3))
 (segment (start 6.35 -33.02) (end 6.35 -22.86) (width 1) (layer F.Cu) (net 4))
 (segment (start 2.54 -22.86) (end 15.24 -22.86) (width 2.2) (layer B.Cu) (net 4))
 (segment (start 6.35 -33.02) (end 15.24 -33.02) (width 2.2) (layer B.Cu) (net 4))
 (segment (start 2.54 -12.7) (end 15.24 -12.7) (width 2.2) (layer B.Cu) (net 5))
 (segment (start 15.24 -7.62) (end 2.54 -7.62) (width 2.2) (layer B.Cu) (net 6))
 (segment (start 8.89 -30.48) (end 8.89 -15.24) (width 1) (layer F.Cu) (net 7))
 (segment (start 2.54 -15.24) (end 15.24 -15.24) (width 2.2) (layer B.Cu) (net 7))
 (segment (start 8.89 -30.48) (end 15.24 -30.48) (width 2.2) (layer B.Cu) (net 7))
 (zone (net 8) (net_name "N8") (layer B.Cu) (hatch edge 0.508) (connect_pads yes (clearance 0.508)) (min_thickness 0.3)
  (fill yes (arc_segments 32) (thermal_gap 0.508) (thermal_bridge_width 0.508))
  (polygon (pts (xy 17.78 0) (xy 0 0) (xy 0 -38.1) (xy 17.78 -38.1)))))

